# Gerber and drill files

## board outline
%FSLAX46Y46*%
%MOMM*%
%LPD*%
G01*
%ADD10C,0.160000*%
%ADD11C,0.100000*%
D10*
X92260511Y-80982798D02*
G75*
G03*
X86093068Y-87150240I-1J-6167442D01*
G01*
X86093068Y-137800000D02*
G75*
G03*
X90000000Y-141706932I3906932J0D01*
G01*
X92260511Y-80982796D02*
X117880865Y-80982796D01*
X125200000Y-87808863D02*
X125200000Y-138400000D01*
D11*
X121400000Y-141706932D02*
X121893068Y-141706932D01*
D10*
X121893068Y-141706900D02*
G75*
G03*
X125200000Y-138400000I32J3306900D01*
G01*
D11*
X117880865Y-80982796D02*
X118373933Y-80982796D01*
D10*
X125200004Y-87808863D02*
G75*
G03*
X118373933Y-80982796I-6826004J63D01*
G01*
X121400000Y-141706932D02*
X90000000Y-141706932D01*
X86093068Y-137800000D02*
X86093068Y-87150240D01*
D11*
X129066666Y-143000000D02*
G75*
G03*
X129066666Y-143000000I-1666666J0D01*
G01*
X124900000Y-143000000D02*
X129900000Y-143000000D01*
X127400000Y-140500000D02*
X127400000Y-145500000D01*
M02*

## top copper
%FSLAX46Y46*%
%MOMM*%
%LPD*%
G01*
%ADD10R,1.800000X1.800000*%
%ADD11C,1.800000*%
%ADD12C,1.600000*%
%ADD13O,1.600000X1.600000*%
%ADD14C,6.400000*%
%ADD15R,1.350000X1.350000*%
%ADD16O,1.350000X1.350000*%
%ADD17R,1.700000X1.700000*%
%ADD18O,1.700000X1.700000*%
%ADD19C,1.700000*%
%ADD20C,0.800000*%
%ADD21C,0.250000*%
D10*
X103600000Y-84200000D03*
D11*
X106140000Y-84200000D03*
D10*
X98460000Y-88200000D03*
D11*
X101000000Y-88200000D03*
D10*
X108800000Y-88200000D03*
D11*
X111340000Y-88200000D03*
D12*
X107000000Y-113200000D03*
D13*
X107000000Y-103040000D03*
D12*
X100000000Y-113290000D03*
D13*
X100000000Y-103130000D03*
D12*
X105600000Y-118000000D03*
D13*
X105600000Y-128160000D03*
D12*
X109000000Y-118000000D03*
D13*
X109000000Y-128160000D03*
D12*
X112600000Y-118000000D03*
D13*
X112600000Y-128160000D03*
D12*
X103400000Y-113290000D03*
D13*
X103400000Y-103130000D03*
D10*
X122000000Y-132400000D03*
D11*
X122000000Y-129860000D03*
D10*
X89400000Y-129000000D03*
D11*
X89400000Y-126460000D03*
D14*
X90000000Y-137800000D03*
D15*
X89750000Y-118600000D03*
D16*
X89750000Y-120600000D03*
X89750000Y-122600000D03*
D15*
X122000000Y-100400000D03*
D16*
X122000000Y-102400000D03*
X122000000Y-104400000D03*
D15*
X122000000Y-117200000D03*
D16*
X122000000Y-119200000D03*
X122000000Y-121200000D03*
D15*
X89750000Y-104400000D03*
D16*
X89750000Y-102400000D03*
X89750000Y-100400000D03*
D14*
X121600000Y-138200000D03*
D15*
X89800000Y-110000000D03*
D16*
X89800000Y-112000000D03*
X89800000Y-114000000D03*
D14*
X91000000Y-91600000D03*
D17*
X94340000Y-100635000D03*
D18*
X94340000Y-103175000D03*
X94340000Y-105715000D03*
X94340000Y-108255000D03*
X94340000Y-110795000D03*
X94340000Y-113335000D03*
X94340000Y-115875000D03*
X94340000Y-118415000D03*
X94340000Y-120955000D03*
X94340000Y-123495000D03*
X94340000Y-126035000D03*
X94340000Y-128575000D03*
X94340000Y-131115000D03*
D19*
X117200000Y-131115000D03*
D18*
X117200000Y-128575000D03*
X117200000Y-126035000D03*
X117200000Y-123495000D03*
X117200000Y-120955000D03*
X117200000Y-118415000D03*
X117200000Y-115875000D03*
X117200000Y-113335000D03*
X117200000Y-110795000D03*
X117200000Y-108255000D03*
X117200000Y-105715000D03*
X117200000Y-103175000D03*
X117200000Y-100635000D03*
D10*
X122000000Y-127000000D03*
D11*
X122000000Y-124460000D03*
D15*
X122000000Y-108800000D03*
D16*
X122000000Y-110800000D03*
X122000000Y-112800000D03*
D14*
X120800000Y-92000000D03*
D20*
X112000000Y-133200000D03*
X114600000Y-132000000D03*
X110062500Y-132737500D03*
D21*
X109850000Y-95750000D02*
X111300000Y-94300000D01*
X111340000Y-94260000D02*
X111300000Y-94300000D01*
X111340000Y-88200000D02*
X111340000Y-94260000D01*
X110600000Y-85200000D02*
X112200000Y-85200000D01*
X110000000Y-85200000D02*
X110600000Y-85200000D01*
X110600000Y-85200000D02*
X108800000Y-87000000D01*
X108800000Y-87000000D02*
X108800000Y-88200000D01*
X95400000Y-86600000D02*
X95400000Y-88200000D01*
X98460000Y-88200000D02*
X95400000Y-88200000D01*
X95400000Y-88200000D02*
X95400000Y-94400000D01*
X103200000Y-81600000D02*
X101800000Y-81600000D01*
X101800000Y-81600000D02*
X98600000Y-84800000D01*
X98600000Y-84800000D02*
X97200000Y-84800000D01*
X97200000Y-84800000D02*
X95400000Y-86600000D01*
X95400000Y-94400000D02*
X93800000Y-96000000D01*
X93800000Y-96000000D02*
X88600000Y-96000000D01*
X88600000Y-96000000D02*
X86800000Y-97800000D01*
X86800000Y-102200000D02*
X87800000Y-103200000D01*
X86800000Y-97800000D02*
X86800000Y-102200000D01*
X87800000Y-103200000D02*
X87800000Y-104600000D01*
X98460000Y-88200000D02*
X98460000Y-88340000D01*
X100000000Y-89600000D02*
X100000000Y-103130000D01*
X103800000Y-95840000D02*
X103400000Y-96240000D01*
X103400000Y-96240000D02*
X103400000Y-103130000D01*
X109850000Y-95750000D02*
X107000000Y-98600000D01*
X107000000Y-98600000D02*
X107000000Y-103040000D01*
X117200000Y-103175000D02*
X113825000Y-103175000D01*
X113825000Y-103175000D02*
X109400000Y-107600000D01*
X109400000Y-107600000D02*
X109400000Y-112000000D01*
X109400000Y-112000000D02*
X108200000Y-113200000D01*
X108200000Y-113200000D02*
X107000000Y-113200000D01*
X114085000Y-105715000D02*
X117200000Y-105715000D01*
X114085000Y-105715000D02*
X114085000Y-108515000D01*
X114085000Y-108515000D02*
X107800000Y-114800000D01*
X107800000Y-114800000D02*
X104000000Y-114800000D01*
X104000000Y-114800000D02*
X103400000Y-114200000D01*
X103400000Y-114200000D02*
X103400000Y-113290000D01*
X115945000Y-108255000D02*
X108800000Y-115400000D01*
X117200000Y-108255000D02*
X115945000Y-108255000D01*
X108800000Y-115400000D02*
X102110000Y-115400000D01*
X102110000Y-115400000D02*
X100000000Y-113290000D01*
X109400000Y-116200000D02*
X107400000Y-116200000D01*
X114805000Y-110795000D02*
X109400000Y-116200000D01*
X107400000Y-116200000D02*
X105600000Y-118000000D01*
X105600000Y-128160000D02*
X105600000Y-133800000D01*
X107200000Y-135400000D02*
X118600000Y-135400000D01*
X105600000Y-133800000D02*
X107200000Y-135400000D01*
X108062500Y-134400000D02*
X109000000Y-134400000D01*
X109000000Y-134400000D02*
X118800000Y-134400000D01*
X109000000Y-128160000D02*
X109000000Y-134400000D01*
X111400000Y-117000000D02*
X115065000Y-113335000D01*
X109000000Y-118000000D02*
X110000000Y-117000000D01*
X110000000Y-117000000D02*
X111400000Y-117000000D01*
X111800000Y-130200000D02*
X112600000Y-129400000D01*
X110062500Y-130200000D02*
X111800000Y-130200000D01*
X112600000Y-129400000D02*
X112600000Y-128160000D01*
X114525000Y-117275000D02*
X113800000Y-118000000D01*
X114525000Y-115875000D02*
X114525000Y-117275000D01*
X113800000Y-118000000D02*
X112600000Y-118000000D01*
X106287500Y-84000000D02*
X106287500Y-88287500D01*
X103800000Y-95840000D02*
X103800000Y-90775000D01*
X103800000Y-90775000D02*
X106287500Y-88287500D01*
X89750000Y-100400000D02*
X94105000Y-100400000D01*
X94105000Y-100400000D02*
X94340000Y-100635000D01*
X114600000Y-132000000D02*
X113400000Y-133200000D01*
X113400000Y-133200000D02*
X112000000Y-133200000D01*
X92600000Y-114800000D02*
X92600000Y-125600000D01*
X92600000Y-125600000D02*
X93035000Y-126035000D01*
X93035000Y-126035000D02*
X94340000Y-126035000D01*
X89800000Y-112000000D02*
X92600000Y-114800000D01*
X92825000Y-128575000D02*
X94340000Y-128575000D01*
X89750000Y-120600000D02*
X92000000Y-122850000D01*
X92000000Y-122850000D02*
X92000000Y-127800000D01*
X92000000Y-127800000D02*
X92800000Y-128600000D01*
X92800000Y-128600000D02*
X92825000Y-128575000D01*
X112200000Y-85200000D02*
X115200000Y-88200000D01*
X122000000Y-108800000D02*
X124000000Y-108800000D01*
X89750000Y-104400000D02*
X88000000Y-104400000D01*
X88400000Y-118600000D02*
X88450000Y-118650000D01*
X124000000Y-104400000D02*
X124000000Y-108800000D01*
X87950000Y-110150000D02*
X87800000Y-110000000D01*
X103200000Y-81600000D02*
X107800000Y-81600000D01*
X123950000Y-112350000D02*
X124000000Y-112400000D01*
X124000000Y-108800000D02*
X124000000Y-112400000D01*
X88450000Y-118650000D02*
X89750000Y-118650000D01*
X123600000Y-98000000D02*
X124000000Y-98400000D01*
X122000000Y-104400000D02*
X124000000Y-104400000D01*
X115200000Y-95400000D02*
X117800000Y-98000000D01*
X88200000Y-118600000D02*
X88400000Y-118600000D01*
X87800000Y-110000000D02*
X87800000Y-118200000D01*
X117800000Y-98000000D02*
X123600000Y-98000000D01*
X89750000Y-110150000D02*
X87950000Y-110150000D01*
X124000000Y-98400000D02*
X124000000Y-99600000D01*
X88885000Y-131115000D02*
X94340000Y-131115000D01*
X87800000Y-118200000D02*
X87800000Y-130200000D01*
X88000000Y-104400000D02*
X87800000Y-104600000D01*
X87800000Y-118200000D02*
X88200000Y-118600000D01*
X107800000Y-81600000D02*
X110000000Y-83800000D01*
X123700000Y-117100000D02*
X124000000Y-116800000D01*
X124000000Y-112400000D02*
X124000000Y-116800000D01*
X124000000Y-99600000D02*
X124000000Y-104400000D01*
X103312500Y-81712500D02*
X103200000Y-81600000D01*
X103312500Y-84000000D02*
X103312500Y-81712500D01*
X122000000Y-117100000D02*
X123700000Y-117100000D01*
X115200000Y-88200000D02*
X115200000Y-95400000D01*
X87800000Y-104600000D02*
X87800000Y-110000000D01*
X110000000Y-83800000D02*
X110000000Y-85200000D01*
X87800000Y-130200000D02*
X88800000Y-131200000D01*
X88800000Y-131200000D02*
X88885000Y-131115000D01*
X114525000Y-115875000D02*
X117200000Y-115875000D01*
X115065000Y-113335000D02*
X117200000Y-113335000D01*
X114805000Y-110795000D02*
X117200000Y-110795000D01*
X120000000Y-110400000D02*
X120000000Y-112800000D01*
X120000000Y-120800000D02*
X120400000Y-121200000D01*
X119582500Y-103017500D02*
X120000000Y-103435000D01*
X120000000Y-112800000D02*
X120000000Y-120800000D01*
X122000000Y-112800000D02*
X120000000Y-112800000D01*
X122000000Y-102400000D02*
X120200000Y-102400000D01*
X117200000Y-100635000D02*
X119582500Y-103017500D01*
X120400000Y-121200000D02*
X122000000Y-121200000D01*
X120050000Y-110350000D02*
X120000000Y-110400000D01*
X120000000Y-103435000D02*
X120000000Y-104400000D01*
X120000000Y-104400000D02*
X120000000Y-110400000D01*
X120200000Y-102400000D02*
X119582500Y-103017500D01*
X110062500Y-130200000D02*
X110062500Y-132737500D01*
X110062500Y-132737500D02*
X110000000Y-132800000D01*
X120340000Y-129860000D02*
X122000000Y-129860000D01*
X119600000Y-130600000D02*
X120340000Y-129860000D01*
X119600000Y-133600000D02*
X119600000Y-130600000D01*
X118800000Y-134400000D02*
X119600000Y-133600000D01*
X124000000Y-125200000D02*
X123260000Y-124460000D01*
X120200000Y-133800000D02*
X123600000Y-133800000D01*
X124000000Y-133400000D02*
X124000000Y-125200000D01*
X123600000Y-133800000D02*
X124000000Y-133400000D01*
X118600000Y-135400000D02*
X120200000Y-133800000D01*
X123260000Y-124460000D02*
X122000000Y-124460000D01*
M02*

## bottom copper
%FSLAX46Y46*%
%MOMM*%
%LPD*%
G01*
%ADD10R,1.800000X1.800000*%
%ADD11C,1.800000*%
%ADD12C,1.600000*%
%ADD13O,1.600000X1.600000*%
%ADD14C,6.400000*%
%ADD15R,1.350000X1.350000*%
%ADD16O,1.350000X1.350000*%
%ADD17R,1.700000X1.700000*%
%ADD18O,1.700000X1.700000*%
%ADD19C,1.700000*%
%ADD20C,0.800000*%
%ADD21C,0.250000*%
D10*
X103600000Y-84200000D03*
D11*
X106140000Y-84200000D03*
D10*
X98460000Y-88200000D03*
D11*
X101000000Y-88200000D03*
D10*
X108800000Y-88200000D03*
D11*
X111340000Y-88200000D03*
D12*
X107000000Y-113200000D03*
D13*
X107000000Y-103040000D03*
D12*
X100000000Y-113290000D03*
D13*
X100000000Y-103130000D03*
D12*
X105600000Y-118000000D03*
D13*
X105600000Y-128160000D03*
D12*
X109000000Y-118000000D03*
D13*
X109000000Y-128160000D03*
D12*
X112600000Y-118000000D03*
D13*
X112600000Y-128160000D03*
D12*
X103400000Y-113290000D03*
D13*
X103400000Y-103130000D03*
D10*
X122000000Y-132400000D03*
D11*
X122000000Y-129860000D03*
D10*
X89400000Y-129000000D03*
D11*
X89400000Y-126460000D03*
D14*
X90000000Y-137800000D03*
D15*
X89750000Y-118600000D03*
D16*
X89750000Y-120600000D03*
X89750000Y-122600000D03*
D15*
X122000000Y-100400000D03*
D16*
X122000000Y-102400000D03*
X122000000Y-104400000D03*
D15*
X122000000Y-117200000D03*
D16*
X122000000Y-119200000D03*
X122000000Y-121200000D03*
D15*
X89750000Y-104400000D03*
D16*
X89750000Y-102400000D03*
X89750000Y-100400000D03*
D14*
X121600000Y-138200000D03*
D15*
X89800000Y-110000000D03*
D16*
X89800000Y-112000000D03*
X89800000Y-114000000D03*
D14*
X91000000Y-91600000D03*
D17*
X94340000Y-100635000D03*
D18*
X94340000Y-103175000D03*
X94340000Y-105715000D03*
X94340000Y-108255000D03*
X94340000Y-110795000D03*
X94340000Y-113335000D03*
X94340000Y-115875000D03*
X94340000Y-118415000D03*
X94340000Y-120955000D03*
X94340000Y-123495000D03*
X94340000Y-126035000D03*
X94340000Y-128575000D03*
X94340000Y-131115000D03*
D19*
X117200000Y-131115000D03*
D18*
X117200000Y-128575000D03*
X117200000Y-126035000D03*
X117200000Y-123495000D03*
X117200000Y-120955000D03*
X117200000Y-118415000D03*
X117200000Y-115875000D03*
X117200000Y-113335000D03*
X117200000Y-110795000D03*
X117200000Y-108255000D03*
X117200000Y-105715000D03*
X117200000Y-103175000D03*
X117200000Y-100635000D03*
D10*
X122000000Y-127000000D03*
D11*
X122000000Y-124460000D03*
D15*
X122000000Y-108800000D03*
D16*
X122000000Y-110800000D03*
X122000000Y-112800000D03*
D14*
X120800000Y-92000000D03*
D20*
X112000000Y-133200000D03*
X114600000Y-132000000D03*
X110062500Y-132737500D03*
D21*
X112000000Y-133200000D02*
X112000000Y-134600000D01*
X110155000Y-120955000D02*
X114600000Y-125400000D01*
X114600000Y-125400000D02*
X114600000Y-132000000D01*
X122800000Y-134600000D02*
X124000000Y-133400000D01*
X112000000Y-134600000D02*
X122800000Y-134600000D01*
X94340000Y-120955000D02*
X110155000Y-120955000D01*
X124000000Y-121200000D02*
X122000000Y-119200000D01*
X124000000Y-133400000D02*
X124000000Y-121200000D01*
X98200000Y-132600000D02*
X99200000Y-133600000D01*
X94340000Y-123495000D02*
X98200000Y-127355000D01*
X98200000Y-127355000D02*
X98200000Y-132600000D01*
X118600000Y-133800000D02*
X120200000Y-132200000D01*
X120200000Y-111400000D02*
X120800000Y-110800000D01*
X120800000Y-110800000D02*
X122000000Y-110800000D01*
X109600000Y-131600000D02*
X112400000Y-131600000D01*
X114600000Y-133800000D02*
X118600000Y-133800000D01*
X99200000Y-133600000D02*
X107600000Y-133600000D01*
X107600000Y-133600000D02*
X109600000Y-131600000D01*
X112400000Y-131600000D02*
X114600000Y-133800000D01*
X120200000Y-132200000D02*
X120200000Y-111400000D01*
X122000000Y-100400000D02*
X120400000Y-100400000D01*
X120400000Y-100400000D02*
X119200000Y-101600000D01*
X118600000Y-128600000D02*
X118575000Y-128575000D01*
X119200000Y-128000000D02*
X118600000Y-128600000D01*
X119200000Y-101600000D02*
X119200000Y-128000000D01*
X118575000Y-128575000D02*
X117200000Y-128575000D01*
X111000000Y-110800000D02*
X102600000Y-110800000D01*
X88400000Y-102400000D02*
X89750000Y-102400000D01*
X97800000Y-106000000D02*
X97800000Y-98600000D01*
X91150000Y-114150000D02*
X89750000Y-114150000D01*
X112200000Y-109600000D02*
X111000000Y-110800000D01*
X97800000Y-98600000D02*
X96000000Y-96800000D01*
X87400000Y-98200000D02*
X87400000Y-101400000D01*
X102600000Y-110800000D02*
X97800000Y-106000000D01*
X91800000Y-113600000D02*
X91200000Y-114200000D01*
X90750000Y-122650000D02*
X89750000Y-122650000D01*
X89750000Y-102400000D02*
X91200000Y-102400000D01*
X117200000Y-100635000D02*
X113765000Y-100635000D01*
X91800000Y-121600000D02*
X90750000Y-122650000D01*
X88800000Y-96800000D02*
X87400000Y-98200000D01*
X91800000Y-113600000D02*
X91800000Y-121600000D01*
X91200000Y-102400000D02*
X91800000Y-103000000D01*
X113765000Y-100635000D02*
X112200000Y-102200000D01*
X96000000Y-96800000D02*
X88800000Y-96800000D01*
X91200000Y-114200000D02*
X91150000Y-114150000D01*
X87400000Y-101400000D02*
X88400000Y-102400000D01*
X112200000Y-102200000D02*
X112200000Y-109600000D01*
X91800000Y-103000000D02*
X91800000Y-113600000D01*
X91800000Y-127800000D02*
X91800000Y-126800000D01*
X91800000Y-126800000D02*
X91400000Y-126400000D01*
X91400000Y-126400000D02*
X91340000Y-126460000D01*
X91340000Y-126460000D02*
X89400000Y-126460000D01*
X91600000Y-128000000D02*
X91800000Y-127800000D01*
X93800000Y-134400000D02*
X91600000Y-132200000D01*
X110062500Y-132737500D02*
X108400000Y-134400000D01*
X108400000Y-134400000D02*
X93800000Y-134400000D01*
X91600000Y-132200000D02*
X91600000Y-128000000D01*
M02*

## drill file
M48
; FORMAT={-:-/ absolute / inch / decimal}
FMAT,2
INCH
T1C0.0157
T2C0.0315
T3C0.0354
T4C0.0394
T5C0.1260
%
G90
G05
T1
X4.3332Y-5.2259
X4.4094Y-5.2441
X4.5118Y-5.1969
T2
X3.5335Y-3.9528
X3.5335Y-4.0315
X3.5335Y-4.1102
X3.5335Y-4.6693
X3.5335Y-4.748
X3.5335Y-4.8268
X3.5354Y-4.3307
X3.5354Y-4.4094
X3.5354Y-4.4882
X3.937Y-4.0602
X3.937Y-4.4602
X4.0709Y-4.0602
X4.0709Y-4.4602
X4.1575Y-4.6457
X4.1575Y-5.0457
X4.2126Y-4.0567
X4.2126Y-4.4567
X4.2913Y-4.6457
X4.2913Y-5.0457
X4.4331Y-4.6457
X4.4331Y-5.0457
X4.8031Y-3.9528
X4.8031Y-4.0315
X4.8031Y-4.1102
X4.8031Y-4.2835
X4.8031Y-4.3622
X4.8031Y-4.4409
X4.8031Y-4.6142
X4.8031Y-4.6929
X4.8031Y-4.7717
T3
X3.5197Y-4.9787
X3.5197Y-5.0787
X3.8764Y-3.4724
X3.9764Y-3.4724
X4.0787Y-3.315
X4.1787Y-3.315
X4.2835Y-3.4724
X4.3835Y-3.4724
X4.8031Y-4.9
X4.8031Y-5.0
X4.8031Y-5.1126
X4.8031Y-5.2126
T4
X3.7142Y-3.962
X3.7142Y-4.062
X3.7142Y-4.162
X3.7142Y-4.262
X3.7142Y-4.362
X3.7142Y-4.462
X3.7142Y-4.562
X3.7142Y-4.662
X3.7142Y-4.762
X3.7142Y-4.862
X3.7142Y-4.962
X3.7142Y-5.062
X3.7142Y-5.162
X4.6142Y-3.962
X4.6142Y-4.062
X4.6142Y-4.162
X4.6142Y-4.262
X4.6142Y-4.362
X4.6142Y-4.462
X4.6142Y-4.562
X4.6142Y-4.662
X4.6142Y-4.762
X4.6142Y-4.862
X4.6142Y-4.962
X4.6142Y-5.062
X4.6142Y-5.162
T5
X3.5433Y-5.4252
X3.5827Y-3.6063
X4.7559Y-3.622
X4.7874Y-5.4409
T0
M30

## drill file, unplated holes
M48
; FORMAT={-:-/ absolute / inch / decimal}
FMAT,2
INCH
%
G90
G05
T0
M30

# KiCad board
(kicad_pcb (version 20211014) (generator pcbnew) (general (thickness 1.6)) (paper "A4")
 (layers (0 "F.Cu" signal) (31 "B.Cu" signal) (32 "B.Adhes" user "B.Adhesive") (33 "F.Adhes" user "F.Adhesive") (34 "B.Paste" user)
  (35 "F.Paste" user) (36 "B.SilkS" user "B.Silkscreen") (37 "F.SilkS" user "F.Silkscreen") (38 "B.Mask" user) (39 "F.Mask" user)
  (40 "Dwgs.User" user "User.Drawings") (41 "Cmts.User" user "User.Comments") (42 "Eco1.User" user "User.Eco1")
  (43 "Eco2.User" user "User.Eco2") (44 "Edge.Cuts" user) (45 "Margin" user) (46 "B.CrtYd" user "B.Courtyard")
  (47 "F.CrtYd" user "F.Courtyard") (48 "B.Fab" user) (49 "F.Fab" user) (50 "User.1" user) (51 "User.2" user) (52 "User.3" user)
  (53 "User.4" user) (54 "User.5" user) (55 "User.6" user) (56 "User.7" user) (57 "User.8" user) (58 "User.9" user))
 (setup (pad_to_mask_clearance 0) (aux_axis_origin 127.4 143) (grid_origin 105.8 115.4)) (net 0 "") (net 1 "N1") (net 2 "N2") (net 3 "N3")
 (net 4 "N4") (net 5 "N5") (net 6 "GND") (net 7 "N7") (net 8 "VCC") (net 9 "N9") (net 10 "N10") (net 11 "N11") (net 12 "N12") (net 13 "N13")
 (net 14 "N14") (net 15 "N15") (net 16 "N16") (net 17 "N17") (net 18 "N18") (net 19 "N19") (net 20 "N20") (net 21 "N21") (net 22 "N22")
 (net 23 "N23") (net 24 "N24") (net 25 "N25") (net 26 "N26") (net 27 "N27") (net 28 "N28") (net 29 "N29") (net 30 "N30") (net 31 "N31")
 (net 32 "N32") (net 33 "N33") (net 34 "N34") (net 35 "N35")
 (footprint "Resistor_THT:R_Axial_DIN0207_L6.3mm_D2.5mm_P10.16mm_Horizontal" (layer "F.Cu") (at 109 118 -90)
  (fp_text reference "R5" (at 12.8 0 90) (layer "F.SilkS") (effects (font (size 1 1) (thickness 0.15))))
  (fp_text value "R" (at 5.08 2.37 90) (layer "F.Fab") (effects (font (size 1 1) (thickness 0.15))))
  (pad "1" thru_hole circle (at 0 0 270) (size 1.6 1.6) (drill 0.8) (layers *.Cu *.Mask) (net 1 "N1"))
  (pad "2" thru_hole oval (at 10.16 0 270) (size 1.6 1.6) (drill 0.8) (layers *.Cu *.Mask) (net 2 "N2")))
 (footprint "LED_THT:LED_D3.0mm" (layer "F.Cu") (at 122 132.4 90)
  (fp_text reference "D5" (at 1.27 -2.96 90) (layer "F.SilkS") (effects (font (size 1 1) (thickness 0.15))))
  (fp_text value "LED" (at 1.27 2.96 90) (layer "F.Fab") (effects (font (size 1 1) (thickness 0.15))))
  (pad "1" thru_hole rect (at 0 0 90) (size 1.8 1.8) (drill 0.9) (layers *.Cu *.Mask) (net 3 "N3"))
  (pad "2" thru_hole circle (at 2.54 0 90) (size 1.8 1.8) (drill 0.9) (layers *.Cu *.Mask) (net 2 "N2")))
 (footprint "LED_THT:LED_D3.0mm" (layer "F.Cu") (at 89.4 129 90)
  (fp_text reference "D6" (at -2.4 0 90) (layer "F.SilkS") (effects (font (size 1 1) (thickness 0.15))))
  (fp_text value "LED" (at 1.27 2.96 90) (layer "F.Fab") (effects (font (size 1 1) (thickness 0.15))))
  (pad "1" thru_hole rect (at 0 0 90) (size 1.8 1.8) (drill 0.9) (layers *.Cu *.Mask) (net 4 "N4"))
  (pad "2" thru_hole circle (at 2.54 0 90) (size 1.8 1.8) (drill 0.9) (layers *.Cu *.Mask) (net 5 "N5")))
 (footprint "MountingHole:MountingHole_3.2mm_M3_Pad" (layer "F.Cu") (at 90 137.8)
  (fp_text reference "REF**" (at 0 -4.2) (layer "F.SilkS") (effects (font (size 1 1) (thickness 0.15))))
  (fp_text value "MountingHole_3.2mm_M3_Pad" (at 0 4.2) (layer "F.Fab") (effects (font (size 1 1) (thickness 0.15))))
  (pad "1" thru_hole circle (at 0 0) (size 6.4 6.4) (drill 3.2) (layers *.Cu *.Mask)))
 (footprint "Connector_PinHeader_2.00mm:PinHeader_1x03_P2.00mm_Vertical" (layer "F.Cu") (at 89.75 118.6)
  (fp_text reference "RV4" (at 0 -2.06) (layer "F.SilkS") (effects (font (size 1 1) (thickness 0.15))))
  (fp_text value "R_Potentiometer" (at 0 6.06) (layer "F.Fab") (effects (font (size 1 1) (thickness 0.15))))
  (pad "1" thru_hole rect (at 0 0) (size 1.35 1.35) (drill 0.8) (layers *.Cu *.Mask) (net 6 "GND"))
  (pad "2" thru_hole oval (at 0 2) (size 1.35 1.35) (drill 0.8) (layers *.Cu *.Mask) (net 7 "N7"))
  (pad "3" thru_hole oval (at 0 4) (size 1.35 1.35) (drill 0.8) (layers *.Cu *.Mask) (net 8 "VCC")))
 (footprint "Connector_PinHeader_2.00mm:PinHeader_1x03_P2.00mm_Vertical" (layer "F.Cu") (at 122 100.4)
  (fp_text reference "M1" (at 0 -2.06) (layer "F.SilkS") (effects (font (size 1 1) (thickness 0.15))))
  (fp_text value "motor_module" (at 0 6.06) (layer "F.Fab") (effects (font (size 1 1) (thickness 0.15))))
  (pad "1" thru_hole rect (at 0 0) (size 1.35 1.35) (drill 0.8) (layers *.Cu *.Mask) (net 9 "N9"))
  (pad "2" thru_hole oval (at 0 2) (size 1.35 1.35) (drill 0.8) (layers *.Cu *.Mask) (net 8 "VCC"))
  (pad "3" thru_hole oval (at 0 4) (size 1.35 1.35) (drill 0.8) (layers *.Cu *.Mask) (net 6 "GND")))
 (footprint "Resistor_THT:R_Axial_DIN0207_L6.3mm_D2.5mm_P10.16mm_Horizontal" (layer "F.Cu") (at 100 113.29 90)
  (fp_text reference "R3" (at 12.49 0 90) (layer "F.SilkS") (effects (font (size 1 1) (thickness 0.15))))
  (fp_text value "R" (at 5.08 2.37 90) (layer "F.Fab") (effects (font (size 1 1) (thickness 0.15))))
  (pad "1" thru_hole circle (at 0 0 90) (size 1.6 1.6) (drill 0.8) (layers *.Cu *.Mask) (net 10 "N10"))
  (pad "2" thru_hole oval (at 10.16 0 90) (size 1.6 1.6) (drill 0.8) (layers *.Cu *.Mask) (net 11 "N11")))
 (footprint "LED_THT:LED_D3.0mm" (layer "F.Cu") (at 98.46 88.2)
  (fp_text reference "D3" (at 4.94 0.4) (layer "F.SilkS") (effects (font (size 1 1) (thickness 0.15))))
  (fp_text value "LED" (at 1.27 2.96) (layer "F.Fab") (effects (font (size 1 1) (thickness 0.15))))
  (pad "1" thru_hole rect (at 0 0) (size 1.8 1.8) (drill 0.9) (layers *.Cu *.Mask) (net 6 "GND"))
  (pad "2" thru_hole circle (at 2.54 0) (size 1.8 1.8) (drill 0.9) (layers *.Cu *.Mask) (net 11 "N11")))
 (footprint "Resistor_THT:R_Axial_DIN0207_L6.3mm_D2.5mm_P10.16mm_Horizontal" (layer "F.Cu") (at 103.4 113.29 90)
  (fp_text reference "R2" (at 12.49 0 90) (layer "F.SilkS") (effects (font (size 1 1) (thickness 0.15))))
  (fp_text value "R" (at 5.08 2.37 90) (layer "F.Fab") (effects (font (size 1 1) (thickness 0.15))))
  (pad "1" thru_hole circle (at 0 0 90) (size 1.6 1.6) (drill 0.8) (layers *.Cu *.Mask) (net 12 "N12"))
  (pad "2" thru_hole oval (at 10.16 0 90) (size 1.6 1.6) (drill 0.8) (layers *.Cu *.Mask) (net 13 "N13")))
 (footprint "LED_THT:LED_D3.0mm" (layer "F.Cu") (at 108.8 88.2)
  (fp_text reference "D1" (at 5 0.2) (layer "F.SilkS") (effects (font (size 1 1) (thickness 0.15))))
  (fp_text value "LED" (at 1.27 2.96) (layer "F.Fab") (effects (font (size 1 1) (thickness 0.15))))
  (pad "1" thru_hole rect (at 0 0) (size 1.8 1.8) (drill 0.9) (layers *.Cu *.Mask) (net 6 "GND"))
  (pad "2" thru_hole circle (at 2.54 0) (size 1.8 1.8) (drill 0.9) (layers *.Cu *.Mask) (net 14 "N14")))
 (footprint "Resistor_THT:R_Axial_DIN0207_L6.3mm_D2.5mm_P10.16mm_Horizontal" (layer "F.Cu") (at 112.6 118 -90)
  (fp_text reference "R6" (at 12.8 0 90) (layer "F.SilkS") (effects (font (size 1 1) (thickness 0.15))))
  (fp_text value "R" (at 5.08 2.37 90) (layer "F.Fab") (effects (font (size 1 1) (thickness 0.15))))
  (pad "1" thru_hole circle (at 0 0 270) (size 1.6 1.6) (drill 0.8) (layers *.Cu *.Mask) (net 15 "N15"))
  (pad "2" thru_hole oval (at 10.16 0 270) (size 1.6 1.6) (drill 0.8) (layers *.Cu *.Mask) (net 5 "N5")))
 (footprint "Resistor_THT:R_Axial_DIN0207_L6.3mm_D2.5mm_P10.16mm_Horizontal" (layer "F.Cu") (at 107 113.2 90)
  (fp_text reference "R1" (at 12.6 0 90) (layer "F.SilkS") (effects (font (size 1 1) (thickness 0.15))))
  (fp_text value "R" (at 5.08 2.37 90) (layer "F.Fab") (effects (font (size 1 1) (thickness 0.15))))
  (pad "1" thru_hole circle (at 0 0 90) (size 1.6 1.6) (drill 0.8) (layers *.Cu *.Mask) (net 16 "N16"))
  (pad "2" thru_hole oval (at 10.16 0 90) (size 1.6 1.6) (drill 0.8) (layers *.Cu *.Mask) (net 14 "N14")))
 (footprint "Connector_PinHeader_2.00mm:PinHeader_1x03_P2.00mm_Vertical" (layer "F.Cu") (at 122 117.2)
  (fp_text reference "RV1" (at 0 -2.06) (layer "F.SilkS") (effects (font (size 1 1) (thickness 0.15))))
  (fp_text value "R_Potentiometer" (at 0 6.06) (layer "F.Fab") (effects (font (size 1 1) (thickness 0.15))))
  (pad "1" thru_hole rect (at 0 0) (size 1.35 1.35) (drill 0.8) (layers *.Cu *.Mask) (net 6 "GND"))
  (pad "2" thru_hole oval (at 0 2) (size 1.35 1.35) (drill 0.8) (layers *.Cu *.Mask) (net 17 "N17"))
  (pad "3" thru_hole oval (at 0 4) (size 1.35 1.35) (drill 0.8) (layers *.Cu *.Mask) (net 8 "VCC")))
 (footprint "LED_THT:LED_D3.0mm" (layer "F.Cu") (at 103.6 84.2)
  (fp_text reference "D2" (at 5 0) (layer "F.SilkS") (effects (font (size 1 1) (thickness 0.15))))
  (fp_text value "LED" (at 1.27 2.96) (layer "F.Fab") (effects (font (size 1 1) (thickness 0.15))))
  (pad "1" thru_hole rect (at 0 0) (size 1.8 1.8) (drill 0.9) (layers *.Cu *.Mask) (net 6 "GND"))
  (pad "2" thru_hole circle (at 2.54 0) (size 1.8 1.8) (drill 0.9) (layers *.Cu *.Mask) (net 13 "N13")))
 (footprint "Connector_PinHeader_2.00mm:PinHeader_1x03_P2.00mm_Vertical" (layer "F.Cu") (at 89.75 104.4 180)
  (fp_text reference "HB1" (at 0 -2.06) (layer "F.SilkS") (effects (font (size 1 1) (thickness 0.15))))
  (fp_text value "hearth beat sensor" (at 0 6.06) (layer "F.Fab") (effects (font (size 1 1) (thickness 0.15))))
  (pad "1" thru_hole rect (at 0 0 180) (size 1.35 1.35) (drill 0.8) (layers *.Cu *.Mask) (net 6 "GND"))
  (pad "2" thru_hole oval (at 0 2 180) (size 1.35 1.35) (drill 0.8) (layers *.Cu *.Mask) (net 8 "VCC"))
  (pad "3" thru_hole oval (at 0 4 180) (size 1.35 1.35) (drill 0.8) (layers *.Cu *.Mask) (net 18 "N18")))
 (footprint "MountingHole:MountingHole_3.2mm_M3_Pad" (layer "F.Cu") (at 121.6 138.2)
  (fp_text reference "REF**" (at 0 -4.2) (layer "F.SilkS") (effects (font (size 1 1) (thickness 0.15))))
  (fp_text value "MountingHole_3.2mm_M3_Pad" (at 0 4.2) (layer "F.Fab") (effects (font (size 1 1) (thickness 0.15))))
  (pad "1" thru_hole circle (at 0 0) (size 6.4 6.4) (drill 3.2) (layers *.Cu *.Mask)))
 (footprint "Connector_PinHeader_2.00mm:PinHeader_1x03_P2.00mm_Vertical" (layer "F.Cu") (at 89.8 110)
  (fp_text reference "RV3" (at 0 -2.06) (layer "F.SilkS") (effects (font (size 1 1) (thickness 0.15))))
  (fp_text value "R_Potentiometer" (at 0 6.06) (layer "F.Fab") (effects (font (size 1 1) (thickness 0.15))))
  (pad "1" thru_hole rect (at 0 0) (size 1.35 1.35) (drill 0.8) (layers *.Cu *.Mask) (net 6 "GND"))
  (pad "2" thru_hole oval (at 0 2) (size 1.35 1.35) (drill 0.8) (layers *.Cu *.Mask) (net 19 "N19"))
  (pad "3" thru_hole oval (at 0 4) (size 1.35 1.35) (drill 0.8) (layers *.Cu *.Mask) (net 8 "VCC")))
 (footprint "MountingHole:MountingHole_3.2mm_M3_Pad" (layer "F.Cu") (at 91 91.6)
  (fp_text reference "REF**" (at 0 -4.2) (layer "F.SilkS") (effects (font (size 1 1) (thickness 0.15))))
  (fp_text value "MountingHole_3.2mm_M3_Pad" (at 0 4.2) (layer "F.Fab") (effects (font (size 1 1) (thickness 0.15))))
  (pad "1" thru_hole circle (at 0 0) (size 6.4 6.4) (drill 3.2) (layers *.Cu *.Mask)))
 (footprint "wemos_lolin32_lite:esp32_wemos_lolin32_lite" (layer "F.Cu") (at 94.34 100.635)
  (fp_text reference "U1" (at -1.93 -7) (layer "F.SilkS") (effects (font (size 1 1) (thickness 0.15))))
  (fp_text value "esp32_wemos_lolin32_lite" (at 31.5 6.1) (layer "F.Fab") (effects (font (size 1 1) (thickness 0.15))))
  (pad "1" thru_hole rect (at 0 0) (size 1.7 1.7) (drill 1) (layers *.Cu *.Mask) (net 18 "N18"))
  (pad "2" thru_hole oval (at 0 2.54) (size 1.7 1.7) (drill 1) (layers *.Cu *.Mask) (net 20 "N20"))
  (pad "3" thru_hole oval (at 0 5.08) (size 1.7 1.7) (drill 1) (layers *.Cu *.Mask) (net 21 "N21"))
  (pad "4" thru_hole oval (at 0 7.62) (size 1.7 1.7) (drill 1) (layers *.Cu *.Mask) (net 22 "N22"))
  (pad "5" thru_hole oval (at 0 10.16) (size 1.7 1.7) (drill 1) (layers *.Cu *.Mask) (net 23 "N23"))
  (pad "6" thru_hole oval (at 0 12.7) (size 1.7 1.7) (drill 1) (layers *.Cu *.Mask) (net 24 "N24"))
  (pad "7" thru_hole oval (at 0 15.24) (size 1.7 1.7) (drill 1) (layers *.Cu *.Mask) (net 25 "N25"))
  (pad "8" thru_hole oval (at 0 17.78) (size 1.7 1.7) (drill 1) (layers *.Cu *.Mask) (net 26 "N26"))
  (pad "9" thru_hole oval (at 0 20.32) (size 1.7 1.7) (drill 1) (layers *.Cu *.Mask) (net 17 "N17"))
  (pad "10" thru_hole oval (at 0 22.86) (size 1.7 1.7) (drill 1) (layers *.Cu *.Mask) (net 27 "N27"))
  (pad "11" thru_hole oval (at 0 25.4) (size 1.7 1.7) (drill 1) (layers *.Cu *.Mask) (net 19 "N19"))
  (pad "12" thru_hole oval (at 0 27.94) (size 1.7 1.7) (drill 1) (layers *.Cu *.Mask) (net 7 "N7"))
  (pad "13" thru_hole oval (at 0 30.48) (size 1.7 1.7) (drill 1) (layers *.Cu *.Mask) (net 6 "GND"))
  (pad "14" thru_hole circle (at 22.86 30.48 180) (size 1.7 1.7) (drill 1) (layers *.Cu *.Mask) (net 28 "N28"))
  (pad "15" thru_hole oval (at 22.86 27.94 180) (size 1.7 1.7) (drill 1) (layers *.Cu *.Mask) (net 9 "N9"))
  (pad "16" thru_hole oval (at 22.86 25.4 180) (size 1.7 1.7) (drill 1) (layers *.Cu *.Mask) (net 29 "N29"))
  (pad "17" thru_hole oval (at 22.86 22.86 180) (size 1.7 1.7) (drill 1) (layers *.Cu *.Mask) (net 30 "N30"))
  (pad "18" thru_hole oval (at 22.86 20.32 180) (size 1.7 1.7) (drill 1) (layers *.Cu *.Mask) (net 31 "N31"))
  (pad "19" thru_hole oval (at 22.86 17.78 180) (size 1.7 1.7) (drill 1) (layers *.Cu *.Mask) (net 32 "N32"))
  (pad "20" thru_hole oval (at 22.86 15.24 180) (size 1.7 1.7) (drill 1) (layers *.Cu *.Mask) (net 15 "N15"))
  (pad "21" thru_hole oval (at 22.86 12.7 180) (size 1.7 1.7) (drill 1) (layers *.Cu *.Mask) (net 1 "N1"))
  (pad "22" thru_hole oval (at 22.86 10.16 180) (size 1.7 1.7) (drill 1) (layers *.Cu *.Mask) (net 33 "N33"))
  (pad "23" thru_hole oval (at 22.86 7.62 180) (size 1.7 1.7) (drill 1) (layers *.Cu *.Mask) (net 10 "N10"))
  (pad "24" thru_hole oval (at 22.86 5.08 180) (size 1.7 1.7) (drill 1) (layers *.Cu *.Mask) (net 12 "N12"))
  (pad "25" thru_hole oval (at 22.86 2.54 180) (size 1.7 1.7) (drill 1) (layers *.Cu *.Mask) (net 16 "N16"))
  (pad "26" thru_hole oval (at 22.86 0 180) (size 1.7 1.7) (drill 1) (layers *.Cu *.Mask) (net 8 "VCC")))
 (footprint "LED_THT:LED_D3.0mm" (layer "F.Cu") (at 122 127 90)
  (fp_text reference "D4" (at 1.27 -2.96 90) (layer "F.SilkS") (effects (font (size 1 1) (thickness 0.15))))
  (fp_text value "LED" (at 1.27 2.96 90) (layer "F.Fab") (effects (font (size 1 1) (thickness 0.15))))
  (pad "1" thru_hole rect (at 0 0 90) (size 1.8 1.8) (drill 0.9) (layers *.Cu *.Mask) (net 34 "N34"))
  (pad "2" thru_hole circle (at 2.54 0 90) (size 1.8 1.8) (drill 0.9) (layers *.Cu *.Mask) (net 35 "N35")))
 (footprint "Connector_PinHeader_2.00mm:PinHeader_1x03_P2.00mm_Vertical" (layer "F.Cu") (at 122 108.8)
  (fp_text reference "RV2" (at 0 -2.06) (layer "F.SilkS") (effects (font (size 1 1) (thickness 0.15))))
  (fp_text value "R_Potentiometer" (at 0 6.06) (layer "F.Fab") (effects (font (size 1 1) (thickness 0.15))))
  (pad "1" thru_hole rect (at 0 0) (size 1.35 1.35) (drill 0.8) (layers *.Cu *.Mask) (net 6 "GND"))
  (pad "2" thru_hole oval (at 0 2) (size 1.35 1.35) (drill 0.8) (layers *.Cu *.Mask) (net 27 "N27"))
  (pad "3" thru_hole oval (at 0 4) (size 1.35 1.35) (drill 0.8) (layers *.Cu *.Mask) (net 8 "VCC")))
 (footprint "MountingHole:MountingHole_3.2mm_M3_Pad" (layer "F.Cu") (at 120.8 92)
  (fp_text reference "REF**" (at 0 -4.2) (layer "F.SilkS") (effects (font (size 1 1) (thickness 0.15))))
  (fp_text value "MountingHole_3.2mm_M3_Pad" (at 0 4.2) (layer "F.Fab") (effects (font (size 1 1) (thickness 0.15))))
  (pad "1" thru_hole circle (at 0 0) (size 6.4 6.4) (drill 3.2) (layers *.Cu *.Mask)))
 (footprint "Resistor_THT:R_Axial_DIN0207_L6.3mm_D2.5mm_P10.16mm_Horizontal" (layer "F.Cu") (at 105.6 118 -90)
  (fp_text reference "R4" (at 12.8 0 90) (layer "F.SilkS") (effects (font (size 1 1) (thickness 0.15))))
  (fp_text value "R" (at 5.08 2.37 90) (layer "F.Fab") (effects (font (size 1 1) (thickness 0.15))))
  (pad "1" thru_hole circle (at 0 0 270) (size 1.6 1.6) (drill 0.8) (layers *.Cu *.Mask) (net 33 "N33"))
  (pad "2" thru_hole oval (at 10.16 0 270) (size 1.6 1.6) (drill 0.8) (layers *.Cu *.Mask) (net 35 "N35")))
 (gr_arc (start 86.093068 87.15024) (mid 87.89947 82.789199) (end 92.260511 80.982796) (layer "Edge.Cuts") (width 0.16))
 (gr_arc (start 90 141.706932) (mid 87.237382 140.562618) (end 86.093068 137.8) (layer "Edge.Cuts") (width 0.16))
 (gr_line (start 92.260511 80.982796) (end 117.880865 80.982796) (layer "Edge.Cuts") (width 0.16))
 (gr_line (start 125.2 87.808863) (end 125.2 138.4) (layer "Edge.Cuts") (width 0.16))
 (gr_line (start 121.4 141.706932) (end 121.893068 141.706932) (layer "Edge.Cuts") (width 0.1))
 (gr_arc (start 125.2 138.4) (mid 124.231422 140.738354) (end 121.893068 141.706932) (layer "Edge.Cuts") (width 0.16))
 (gr_line (start 117.880865 80.982796) (end 118.373933 80.982796) (layer "Edge.Cuts") (width 0.1))
 (gr_arc (start 118.373933 80.982796) (mid 123.200727 82.98209) (end 125.2 87.808863) (layer "Edge.Cuts") (width 0.16))
 (gr_line (start 121.4 141.706932) (end 90 141.706932) (layer "Edge.Cuts") (width 0.16))
 (gr_line (start 86.093068 137.8) (end 86.093068 87.15024) (layer "Edge.Cuts") (width 0.16))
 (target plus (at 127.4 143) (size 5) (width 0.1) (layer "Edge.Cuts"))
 (segment (start 89.75 100.4) (end 94.105 100.4) (width 0.25) (layer "F.Cu") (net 18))
 (segment (start 94.105 100.4) (end 94.34 100.635) (width 0.25) (layer "F.Cu") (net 18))
 (segment (start 114.6 132) (end 113.4 133.2) (width 0.25) (layer "F.Cu") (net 17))
 (segment (start 113.4 133.2) (end 112 133.2) (width 0.25) (layer "F.Cu") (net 17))
 (via (at 112 133.2) (size 0.8) (drill 0.4) (layers "F.Cu" "B.Cu") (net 17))
 (via (at 114.6 132) (size 0.8) (drill 0.4) (layers "F.Cu" "B.Cu") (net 17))
 (segment (start 112 133.2) (end 112 134.6) (width 0.25) (layer "B.Cu") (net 17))
 (segment (start 110.155 120.955) (end 114.6 125.4) (width 0.25) (layer "B.Cu") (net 17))
 (segment (start 114.6 125.4) (end 114.6 132) (width 0.25) (layer "B.Cu") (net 17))
 (segment (start 122.8 134.6) (end 124 133.4) (width 0.25) (layer "B.Cu") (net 17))
 (segment (start 112 134.6) (end 122.8 134.6) (width 0.25) (layer "B.Cu") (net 17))
 (segment (start 94.34 120.955) (end 110.155 120.955) (width 0.25) (layer "B.Cu") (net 17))
 (segment (start 124 121.2) (end 122 119.2) (width 0.25) (layer "B.Cu") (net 17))
 (segment (start 124 133.4) (end 124 121.2) (width 0.25) (layer "B.Cu") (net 17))
 (segment (start 98.2 132.6) (end 99.2 133.6) (width 0.25) (layer "B.Cu") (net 27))
 (segment (start 94.34 123.495) (end 98.2 127.355) (width 0.25) (layer "B.Cu") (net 27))
 (segment (start 98.2 127.355) (end 98.2 132.6) (width 0.25) (layer "B.Cu") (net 27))
 (segment (start 118.6 133.8) (end 120.2 132.2) (width 0.25) (layer "B.Cu") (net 27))
 (segment (start 120.2 111.4) (end 120.8 110.8) (width 0.25) (layer "B.Cu") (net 27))
 (segment (start 120.8 110.8) (end 122 110.8) (width 0.25) (layer "B.Cu") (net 27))
 (segment (start 109.6 131.6) (end 112.4 131.6) (width 0.25) (layer "B.Cu") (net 27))
 (segment (start 114.6 133.8) (end 118.6 133.8) (width 0.25) (layer "B.Cu") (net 27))
 (segment (start 99.2 133.6) (end 107.6 133.6) (width 0.25) (layer "B.Cu") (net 27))
 (segment (start 107.6 133.6) (end 109.6 131.6) (width 0.25) (layer "B.Cu") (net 27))
 (segment (start 112.4 131.6) (end 114.6 133.8) (width 0.25) (layer "B.Cu") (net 27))
 (segment (start 120.2 132.2) (end 120.2 111.4) (width 0.25) (layer "B.Cu") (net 27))
 (segment (start 92.6 114.8) (end 92.6 125.6) (width 0.25) (layer "F.Cu") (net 19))
 (segment (start 92.6 125.6) (end 93.035 126.035) (width 0.25) (layer "F.Cu") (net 19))
 (segment (start 93.035 126.035) (end 94.34 126.035) (width 0.25) (layer "F.Cu") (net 19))
 (segment (start 89.8 112) (end 92.6 114.8) (width 0.25) (layer "F.Cu") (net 19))
 (segment (start 92.825 128.575) (end 94.34 128.575) (width 0.25) (layer "F.Cu") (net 7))
 (segment (start 89.75 120.6) (end 92 122.85) (width 0.25) (layer "F.Cu") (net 7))
 (segment (start 92 122.85) (end 92 127.8) (width 0.25) (layer "F.Cu") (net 7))
 (segment (start 92 127.8) (end 92.8 128.6) (width 0.25) (layer "F.Cu") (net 7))
 (segment (start 92.8 128.6) (end 92.825 128.575) (width 0.25) (layer "F.Cu") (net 7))
 (segment (start 95.4 86.6) (end 95.4 88.2) (width 0.25) (layer "F.Cu") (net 6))
 (segment (start 86.8 97.8) (end 86.8 102.2) (width 0.25) (layer "F.Cu") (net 6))
 (segment (start 112.2 85.2) (end 115.2 88.2) (width 0.25) (layer "F.Cu") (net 6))
 (segment (start 122 108.8) (end 124 108.8) (width 0.25) (layer "F.Cu") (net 6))
 (segment (start 89.75 104.4) (end 88 104.4) (width 0.25) (layer "F.Cu") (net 6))
 (segment (start 88.4 118.6) (end 88.45 118.65) (width 0.25) (layer "F.Cu") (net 6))
 (segment (start 110.6 85.2) (end 108.8 87) (width 0.25) (layer "F.Cu") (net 6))
 (segment (start 124 104.4) (end 124 108.8) (width 0.25) (layer "F.Cu") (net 6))
 (segment (start 87.95 110.15) (end 87.8 110) (width 0.25) (layer "F.Cu") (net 6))
 (segment (start 103.2 81.6) (end 107.8 81.6) (width 0.25) (layer "F.Cu") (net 6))
 (segment (start 123.95 112.35) (end 124 112.4) (width 0.25) (layer "F.Cu") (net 6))
 (segment (start 124 108.8) (end 124 112.4) (width 0.25) (layer "F.Cu") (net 6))
 (segment (start 93.8 96) (end 88.6 96) (width 0.25) (layer "F.Cu") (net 6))
 (segment (start 88.45 118.65) (end 89.75 118.65) (width 0.25) (layer "F.Cu") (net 6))
 (segment (start 123.6 98) (end 124 98.4) (width 0.25) (layer "F.Cu") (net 6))
 (segment (start 122 104.4) (end 124 104.4) (width 0.25) (layer "F.Cu") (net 6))
 (segment (start 101.8 81.6) (end 98.6 84.8) (width 0.25) (layer "F.Cu") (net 6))
 (segment (start 115.2 95.4) (end 117.8 98) (width 0.25) (layer "F.Cu") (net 6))
 (segment (start 88.2 118.6) (end 88.4 118.6) (width 0.25) (layer "F.Cu") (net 6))
 (segment (start 87.8 110) (end 87.8 118.2) (width 0.25) (layer "F.Cu") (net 6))
 (segment (start 87.8 103.2) (end 87.8 104.6) (width 0.25) (layer "F.Cu") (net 6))
 (segment (start 117.8 98) (end 123.6 98) (width 0.25) (layer "F.Cu") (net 6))
 (segment (start 89.75 110.15) (end 87.95 110.15) (width 0.25) (layer "F.Cu") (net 6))
 (segment (start 110 85.2) (end 110.6 85.2) (width 0.25) (layer "F.Cu") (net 6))
 (segment (start 95.4 94.4) (end 93.8 96) (width 0.25) (layer "F.Cu") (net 6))
 (segment (start 124 98.4) (end 124 99.6) (width 0.25) (layer "F.Cu") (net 6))
 (segment (start 88.6 96) (end 86.8 97.8) (width 0.25) (layer "F.Cu") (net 6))
 (segment (start 88.885 131.115) (end 94.34 131.115) (width 0.25) (layer "F.Cu") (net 6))
 (segment (start 87.8 118.2) (end 87.8 130.2) (width 0.25) (layer "F.Cu") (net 6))
 (segment (start 95.4 88.2) (end 95.4 94.4) (width 0.25) (layer "F.Cu") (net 6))
 (segment (start 88 104.4) (end 87.8 104.6) (width 0.25) (layer "F.Cu") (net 6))
 (segment (start 97.2 84.8) (end 95.4 86.6) (width 0.25) (layer "F.Cu") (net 6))
 (segment (start 87.8 118.2) (end 88.2 118.6) (width 0.25) (layer "F.Cu") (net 6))
 (segment (start 107.8 81.6) (end 110 83.8) (width 0.25) (layer "F.Cu") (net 6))
 (segment (start 98.46 88.2) (end 95.4 88.2) (width 0.25) (layer "F.Cu") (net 6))
 (segment (start 123.7 117.1) (end 124 116.8) (width 0.25) (layer "F.Cu") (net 6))
 (segment (start 98.6 84.8) (end 97.2 84.8) (width 0.25) (layer "F.Cu") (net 6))
 (segment (start 86.8 102.2) (end 87.8 103.2) (width 0.25) (layer "F.Cu") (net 6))
 (segment (start 124 112.4) (end 124 116.8) (width 0.25) (layer "F.Cu") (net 6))
 (segment (start 124 99.6) (end 124 104.4) (width 0.25) (layer "F.Cu") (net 6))
 (segment (start 103.3125 81.7125) (end 103.2 81.6) (width 0.25) (layer "F.Cu") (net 6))
 (segment (start 103.2 81.6) (end 101.8 81.6) (width 0.25) (layer "F.Cu") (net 6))
 (segment (start 108.8 87) (end 108.8 88.2) (width 0.25) (layer "F.Cu") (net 6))
 (segment (start 103.3125 84) (end 103.3125 81.7125) (width 0.25) (layer "F.Cu") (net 6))
 (segment (start 110.6 85.2) (end 112.2 85.2) (width 0.25) (layer "F.Cu") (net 6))
 (segment (start 122 117.1) (end 123.7 117.1) (width 0.25) (layer "F.Cu") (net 6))
 (segment (start 98.46 88.2) (end 98.46 88.34) (width 0.25) (layer "F.Cu") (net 6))
 (segment (start 115.2 88.2) (end 115.2 95.4) (width 0.25) (layer "F.Cu") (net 6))
 (segment (start 87.8 104.6) (end 87.8 110) (width 0.25) (layer "F.Cu") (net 6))
 (segment (start 110 83.8) (end 110 85.2) (width 0.25) (layer "F.Cu") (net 6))
 (segment (start 87.8 130.2) (end 88.8 131.2) (width 0.25) (layer "F.Cu") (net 6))
 (segment (start 88.8 131.2) (end 88.885 131.115) (width 0.25) (layer "F.Cu") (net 6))
 (segment (start 122 100.4) (end 120.4 100.4) (width 0.25) (layer "B.Cu") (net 9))
 (segment (start 120.4 100.4) (end 119.2 101.6) (width 0.25) (layer "B.Cu") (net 9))
 (segment (start 118.6 128.6) (end 118.575 128.575) (width 0.25) (layer "B.Cu") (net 9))
 (segment (start 119.2 128) (end 118.6 128.6) (width 0.25) (layer "B.Cu") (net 9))
 (segment (start 119.2 101.6) (end 119.2 128) (width 0.25) (layer "B.Cu") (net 9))
 (segment (start 118.575 128.575) (end 117.2 128.575) (width 0.25) (layer "B.Cu") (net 9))
 (segment (start 114.525 115.875) (end 117.2 115.875) (width 0.25) (layer "F.Cu") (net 15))
 (segment (start 113.8 118) (end 112.6 118) (width 0.25) (layer "F.Cu") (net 15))
 (segment (start 114.525 115.875) (end 114.525 117.275) (width 0.25) (layer "F.Cu") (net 15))
 (segment (start 114.525 117.275) (end 113.8 118) (width 0.25) (layer "F.Cu") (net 15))
 (segment (start 110 117) (end 111.4 117) (width 0.25) (layer "F.Cu") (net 1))
 (segment (start 111.4 117) (end 115.065 113.335) (width 0.25) (layer "F.Cu") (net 1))
 (segment (start 115.065 113.335) (end 117.2 113.335) (width 0.25) (layer "F.Cu") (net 1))
 (segment (start 109 118) (end 110 117) (width 0.25) (layer "F.Cu") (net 1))
 (segment (start 114.805 110.795) (end 109.4 116.2) (width 0.25) (layer "F.Cu") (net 33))
 (segment (start 107.4 116.2) (end 105.6 118) (width 0.25) (layer "F.Cu") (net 33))
 (segment (start 109.4 116.2) (end 107.4 116.2) (width 0.25) (layer "F.Cu") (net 33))
 (segment (start 114.805 110.795) (end 117.2 110.795) (width 0.25) (layer "F.Cu") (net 33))
 (segment (start 102.11 115.4) (end 100 113.29) (width 0.25) (layer "F.Cu") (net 10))
 (segment (start 117.2 108.255) (end 115.945 108.255) (width 0.25) (layer "F.Cu") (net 10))
 (segment (start 115.945 108.255) (end 108.8 115.4) (width 0.25) (layer "F.Cu") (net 10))
 (segment (start 108.8 115.4) (end 102.11 115.4) (width 0.25) (layer "F.Cu") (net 10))
 (segment (start 103.4 114.2) (end 103.4 113.29) (width 0.25) (layer "F.Cu") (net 12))
 (segment (start 114.085 105.715) (end 117.2 105.715) (width 0.25) (layer "F.Cu") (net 12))
 (segment (start 114.085 108.515) (end 107.8 114.8) (width 0.25) (layer "F.Cu") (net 12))
 (segment (start 107.8 114.8) (end 104 114.8) (width 0.25) (layer "F.Cu") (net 12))
 (segment (start 104 114.8) (end 103.4 114.2) (width 0.25) (layer "F.Cu") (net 12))
 (segment (start 114.085 105.715) (end 114.085 108.515) (width 0.25) (layer "F.Cu") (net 12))
 (segment (start 117.2 103.175) (end 113.825 103.175) (width 0.25) (layer "F.Cu") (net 16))
 (segment (start 109.4 107.6) (end 109.4 112) (width 0.25) (layer "F.Cu") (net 16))
 (segment (start 113.825 103.175) (end 109.4 107.6) (width 0.25) (layer "F.Cu") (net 16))
 (segment (start 108.2 113.2) (end 107 113.2) (width 0.25) (layer "F.Cu") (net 16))
 (segment (start 109.4 112) (end 108.2 113.2) (width 0.25) (layer "F.Cu") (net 16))
 (segment (start 120 110.4) (end 120 112.8) (width 0.25) (layer "F.Cu") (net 8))
 (segment (start 120 120.8) (end 120.4 121.2) (width 0.25) (layer "F.Cu") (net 8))
 (segment (start 119.5825 103.0175) (end 120 103.435) (width 0.25) (layer "F.Cu") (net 8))
 (segment (start 120 112.8) (end 120 120.8) (width 0.25) (layer "F.Cu") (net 8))
 (segment (start 122 112.8) (end 120 112.8) (width 0.25) (layer "F.Cu") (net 8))
 (segment (start 122 102.4) (end 120.2 102.4) (width 0.25) (layer "F.Cu") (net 8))
 (segment (start 117.2 100.635) (end 119.5825 103.0175) (width 0.25) (layer "F.Cu") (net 8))
 (segment (start 120.4 121.2) (end 122 121.2) (width 0.25) (layer "F.Cu") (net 8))
 (segment (start 120.05 110.35) (end 120 110.4) (width 0.25) (layer "F.Cu") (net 8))
 (segment (start 120 103.435) (end 120 104.4) (width 0.25) (layer "F.Cu") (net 8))
 (segment (start 120 104.4) (end 120 110.4) (width 0.25) (layer "F.Cu") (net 8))
 (segment (start 120.2 102.4) (end 119.5825 103.0175) (width 0.25) (layer "F.Cu") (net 8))
 (segment (start 111 110.8) (end 102.6 110.8) (width 0.25) (layer "B.Cu") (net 8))
 (segment (start 88.4 102.4) (end 89.75 102.4) (width 0.25) (layer "B.Cu") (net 8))
 (segment (start 97.8 106) (end 97.8 98.6) (width 0.25) (layer "B.Cu") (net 8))
 (segment (start 91.15 114.15) (end 89.75 114.15) (width 0.25) (layer "B.Cu") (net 8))
 (segment (start 112.2 109.6) (end 111 110.8) (width 0.25) (layer "B.Cu") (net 8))
 (segment (start 97.8 98.6) (end 96 96.8) (width 0.25) (layer "B.Cu") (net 8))
 (segment (start 87.4 98.2) (end 87.4 101.4) (width 0.25) (layer "B.Cu") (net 8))
 (segment (start 102.6 110.8) (end 97.8 106) (width 0.25) (layer "B.Cu") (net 8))
 (segment (start 91.8 113.6) (end 91.2 114.2) (width 0.25) (layer "B.Cu") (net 8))
 (segment (start 90.75 122.65) (end 89.75 122.65) (width 0.25) (layer "B.Cu") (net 8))
 (segment (start 89.75 102.4) (end 91.2 102.4) (width 0.25) (layer "B.Cu") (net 8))
 (segment (start 117.2 100.635) (end 113.765 100.635) (width 0.25) (layer "B.Cu") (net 8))
 (segment (start 91.8 121.6) (end 90.75 122.65) (width 0.25) (layer "B.Cu") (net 8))
 (segment (start 88.8 96.8) (end 87.4 98.2) (width 0.25) (layer "B.Cu") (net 8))
 (segment (start 91.8 113.6) (end 91.8 121.6) (width 0.25) (layer "B.Cu") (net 8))
 (segment (start 91.2 102.4) (end 91.8 103) (width 0.25) (layer "B.Cu") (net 8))
 (segment (start 113.765 100.635) (end 112.2 102.2) (width 0.25) (layer "B.Cu") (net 8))
 (segment (start 96 96.8) (end 88.8 96.8) (width 0.25) (layer "B.Cu") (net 8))
 (segment (start 91.2 114.2) (end 91.15 114.15) (width 0.25) (layer "B.Cu") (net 8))
 (segment (start 87.4 101.4) (end 88.4 102.4) (width 0.25) (layer "B.Cu") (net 8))
 (segment (start 112.2 102.2) (end 112.2 109.6) (width 0.25) (layer "B.Cu") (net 8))
 (segment (start 91.8 103) (end 91.8 113.6) (width 0.25) (layer "B.Cu") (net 8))
 (segment (start 111.34 94.26) (end 111.3 94.3) (width 0.25) (layer "F.Cu") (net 14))
 (segment (start 111.34 88.2) (end 111.34 94.26) (width 0.25) (layer "F.Cu") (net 14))
 (segment (start 109.85 95.75) (end 111.3 94.3) (width 0.25) (layer "F.Cu") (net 14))
 (segment (start 107 98.6) (end 107 103.04) (width 0.25) (layer "F.Cu") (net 14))
 (segment (start 109.85 95.75) (end 107 98.6) (width 0.25) (layer "F.Cu") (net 14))
 (segment (start 106.2875 84) (end 106.2875 88.2875) (width 0.25) (layer "F.Cu") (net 13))
 (segment (start 103.8 90.775) (end 106.2875 88.2875) (width 0.25) (layer "F.Cu") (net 13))
 (segment (start 103.4 96.24) (end 103.4 103.13) (width 0.25) (layer "F.Cu") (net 13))
 (segment (start 103.8 95.84) (end 103.4 96.24) (width 0.25) (layer "F.Cu") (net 13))
 (segment (start 103.8 95.84) (end 103.8 90.775) (width 0.25) (layer "F.Cu") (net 13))
 (segment (start 100 89.6) (end 100 103.13) (width 0.25) (layer "F.Cu") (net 11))
 (segment (start 111.8 130.2) (end 112.6 129.4) (width 0.25) (layer "F.Cu") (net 5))
 (segment (start 110.0625 130.2) (end 111.8 130.2) (width 0.25) (layer "F.Cu") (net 5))
 (segment (start 110.0625 130.2) (end 110.0625 132.7375) (width 0.25) (layer "F.Cu") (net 5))
 (segment (start 110.0625 132.7375) (end 110 132.8) (width 0.25) (layer "F.Cu") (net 5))
 (segment (start 112.6 129.4) (end 112.6 128.16) (width 0.25) (layer "F.Cu") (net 5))
 (via (at 110.0625 132.7375) (size 0.8) (drill 0.4) (layers "F.Cu" "B.Cu") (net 5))
 (segment (start 91.8 127.8) (end 91.8 126.8) (width 0.25) (layer "B.Cu") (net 5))
 (segment (start 91.8 126.8) (end 91.4 126.4) (width 0.25) (layer "B.Cu") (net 5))
 (segment (start 91.4 126.4) (end 91.34 126.46) (width 0.25) (layer "B.Cu") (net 5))
 (segment (start 91.34 126.46) (end 89.4 126.46) (width 0.25) (layer "B.Cu") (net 5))
 (segment (start 91.6 128) (end 91.8 127.8) (width 0.25) (layer "B.Cu") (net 5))
 (segment (start 93.8 134.4) (end 91.6 132.2) (width 0.25) (layer "B.Cu") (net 5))
 (segment (start 110.0625 132.7375) (end 108.4 134.4) (width 0.25) (layer "B.Cu") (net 5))
 (segment (start 108.4 134.4) (end 93.8 134.4) (width 0.25) (layer "B.Cu") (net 5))
 (segment (start 91.6 132.2) (end 91.6 128) (width 0.25) (layer "B.Cu") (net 5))
 (segment (start 120.34 129.86) (end 122 129.86) (width 0.25) (layer "F.Cu") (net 2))
 (segment (start 108.0625 134.4) (end 109 134.4) (width 0.25) (layer "F.Cu") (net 2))
 (segment (start 109 134.4) (end 118.8 134.4) (width 0.25) (layer "F.Cu") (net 2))
 (segment (start 119.6 130.6) (end 120.34 129.86) (width 0.25) (layer "F.Cu") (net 2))
 (segment (start 109 128.16) (end 109 134.4) (width 0.25) (layer "F.Cu") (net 2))
 (segment (start 119.6 133.6) (end 119.6 130.6) (width 0.25) (layer "F.Cu") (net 2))
 (segment (start 118.8 134.4) (end 119.6 133.6) (width 0.25) (layer "F.Cu") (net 2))
 (segment (start 107.2 135.4) (end 118.6 135.4) (width 0.25) (layer "F.Cu") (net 35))
 (segment (start 105.6 128.16) (end 105.6 133.8) (width 0.25) (layer "F.Cu") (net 35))
 (segment (start 124 125.2) (end 123.26 124.46) (width 0.25) (layer "F.Cu") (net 35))
 (segment (start 120.2 133.8) (end 123.6 133.8) (width 0.25) (layer "F.Cu") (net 35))
 (segment (start 105.6 133.8) (end 107.2 135.4) (width 0.25) (layer "F.Cu") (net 35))
 (segment (start 124 133.4) (end 124 125.2) (width 0.25) (layer "F.Cu") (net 35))
 (segment (start 123.6 133.8) (end 124 133.4) (width 0.25) (layer "F.Cu") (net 35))
 (segment (start 118.6 135.4) (end 120.2 133.8) (width 0.25) (layer "F.Cu") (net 35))
 (segment (start 123.26 124.46) (end 122 124.46) (width 0.25) (layer "F.Cu") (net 35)))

